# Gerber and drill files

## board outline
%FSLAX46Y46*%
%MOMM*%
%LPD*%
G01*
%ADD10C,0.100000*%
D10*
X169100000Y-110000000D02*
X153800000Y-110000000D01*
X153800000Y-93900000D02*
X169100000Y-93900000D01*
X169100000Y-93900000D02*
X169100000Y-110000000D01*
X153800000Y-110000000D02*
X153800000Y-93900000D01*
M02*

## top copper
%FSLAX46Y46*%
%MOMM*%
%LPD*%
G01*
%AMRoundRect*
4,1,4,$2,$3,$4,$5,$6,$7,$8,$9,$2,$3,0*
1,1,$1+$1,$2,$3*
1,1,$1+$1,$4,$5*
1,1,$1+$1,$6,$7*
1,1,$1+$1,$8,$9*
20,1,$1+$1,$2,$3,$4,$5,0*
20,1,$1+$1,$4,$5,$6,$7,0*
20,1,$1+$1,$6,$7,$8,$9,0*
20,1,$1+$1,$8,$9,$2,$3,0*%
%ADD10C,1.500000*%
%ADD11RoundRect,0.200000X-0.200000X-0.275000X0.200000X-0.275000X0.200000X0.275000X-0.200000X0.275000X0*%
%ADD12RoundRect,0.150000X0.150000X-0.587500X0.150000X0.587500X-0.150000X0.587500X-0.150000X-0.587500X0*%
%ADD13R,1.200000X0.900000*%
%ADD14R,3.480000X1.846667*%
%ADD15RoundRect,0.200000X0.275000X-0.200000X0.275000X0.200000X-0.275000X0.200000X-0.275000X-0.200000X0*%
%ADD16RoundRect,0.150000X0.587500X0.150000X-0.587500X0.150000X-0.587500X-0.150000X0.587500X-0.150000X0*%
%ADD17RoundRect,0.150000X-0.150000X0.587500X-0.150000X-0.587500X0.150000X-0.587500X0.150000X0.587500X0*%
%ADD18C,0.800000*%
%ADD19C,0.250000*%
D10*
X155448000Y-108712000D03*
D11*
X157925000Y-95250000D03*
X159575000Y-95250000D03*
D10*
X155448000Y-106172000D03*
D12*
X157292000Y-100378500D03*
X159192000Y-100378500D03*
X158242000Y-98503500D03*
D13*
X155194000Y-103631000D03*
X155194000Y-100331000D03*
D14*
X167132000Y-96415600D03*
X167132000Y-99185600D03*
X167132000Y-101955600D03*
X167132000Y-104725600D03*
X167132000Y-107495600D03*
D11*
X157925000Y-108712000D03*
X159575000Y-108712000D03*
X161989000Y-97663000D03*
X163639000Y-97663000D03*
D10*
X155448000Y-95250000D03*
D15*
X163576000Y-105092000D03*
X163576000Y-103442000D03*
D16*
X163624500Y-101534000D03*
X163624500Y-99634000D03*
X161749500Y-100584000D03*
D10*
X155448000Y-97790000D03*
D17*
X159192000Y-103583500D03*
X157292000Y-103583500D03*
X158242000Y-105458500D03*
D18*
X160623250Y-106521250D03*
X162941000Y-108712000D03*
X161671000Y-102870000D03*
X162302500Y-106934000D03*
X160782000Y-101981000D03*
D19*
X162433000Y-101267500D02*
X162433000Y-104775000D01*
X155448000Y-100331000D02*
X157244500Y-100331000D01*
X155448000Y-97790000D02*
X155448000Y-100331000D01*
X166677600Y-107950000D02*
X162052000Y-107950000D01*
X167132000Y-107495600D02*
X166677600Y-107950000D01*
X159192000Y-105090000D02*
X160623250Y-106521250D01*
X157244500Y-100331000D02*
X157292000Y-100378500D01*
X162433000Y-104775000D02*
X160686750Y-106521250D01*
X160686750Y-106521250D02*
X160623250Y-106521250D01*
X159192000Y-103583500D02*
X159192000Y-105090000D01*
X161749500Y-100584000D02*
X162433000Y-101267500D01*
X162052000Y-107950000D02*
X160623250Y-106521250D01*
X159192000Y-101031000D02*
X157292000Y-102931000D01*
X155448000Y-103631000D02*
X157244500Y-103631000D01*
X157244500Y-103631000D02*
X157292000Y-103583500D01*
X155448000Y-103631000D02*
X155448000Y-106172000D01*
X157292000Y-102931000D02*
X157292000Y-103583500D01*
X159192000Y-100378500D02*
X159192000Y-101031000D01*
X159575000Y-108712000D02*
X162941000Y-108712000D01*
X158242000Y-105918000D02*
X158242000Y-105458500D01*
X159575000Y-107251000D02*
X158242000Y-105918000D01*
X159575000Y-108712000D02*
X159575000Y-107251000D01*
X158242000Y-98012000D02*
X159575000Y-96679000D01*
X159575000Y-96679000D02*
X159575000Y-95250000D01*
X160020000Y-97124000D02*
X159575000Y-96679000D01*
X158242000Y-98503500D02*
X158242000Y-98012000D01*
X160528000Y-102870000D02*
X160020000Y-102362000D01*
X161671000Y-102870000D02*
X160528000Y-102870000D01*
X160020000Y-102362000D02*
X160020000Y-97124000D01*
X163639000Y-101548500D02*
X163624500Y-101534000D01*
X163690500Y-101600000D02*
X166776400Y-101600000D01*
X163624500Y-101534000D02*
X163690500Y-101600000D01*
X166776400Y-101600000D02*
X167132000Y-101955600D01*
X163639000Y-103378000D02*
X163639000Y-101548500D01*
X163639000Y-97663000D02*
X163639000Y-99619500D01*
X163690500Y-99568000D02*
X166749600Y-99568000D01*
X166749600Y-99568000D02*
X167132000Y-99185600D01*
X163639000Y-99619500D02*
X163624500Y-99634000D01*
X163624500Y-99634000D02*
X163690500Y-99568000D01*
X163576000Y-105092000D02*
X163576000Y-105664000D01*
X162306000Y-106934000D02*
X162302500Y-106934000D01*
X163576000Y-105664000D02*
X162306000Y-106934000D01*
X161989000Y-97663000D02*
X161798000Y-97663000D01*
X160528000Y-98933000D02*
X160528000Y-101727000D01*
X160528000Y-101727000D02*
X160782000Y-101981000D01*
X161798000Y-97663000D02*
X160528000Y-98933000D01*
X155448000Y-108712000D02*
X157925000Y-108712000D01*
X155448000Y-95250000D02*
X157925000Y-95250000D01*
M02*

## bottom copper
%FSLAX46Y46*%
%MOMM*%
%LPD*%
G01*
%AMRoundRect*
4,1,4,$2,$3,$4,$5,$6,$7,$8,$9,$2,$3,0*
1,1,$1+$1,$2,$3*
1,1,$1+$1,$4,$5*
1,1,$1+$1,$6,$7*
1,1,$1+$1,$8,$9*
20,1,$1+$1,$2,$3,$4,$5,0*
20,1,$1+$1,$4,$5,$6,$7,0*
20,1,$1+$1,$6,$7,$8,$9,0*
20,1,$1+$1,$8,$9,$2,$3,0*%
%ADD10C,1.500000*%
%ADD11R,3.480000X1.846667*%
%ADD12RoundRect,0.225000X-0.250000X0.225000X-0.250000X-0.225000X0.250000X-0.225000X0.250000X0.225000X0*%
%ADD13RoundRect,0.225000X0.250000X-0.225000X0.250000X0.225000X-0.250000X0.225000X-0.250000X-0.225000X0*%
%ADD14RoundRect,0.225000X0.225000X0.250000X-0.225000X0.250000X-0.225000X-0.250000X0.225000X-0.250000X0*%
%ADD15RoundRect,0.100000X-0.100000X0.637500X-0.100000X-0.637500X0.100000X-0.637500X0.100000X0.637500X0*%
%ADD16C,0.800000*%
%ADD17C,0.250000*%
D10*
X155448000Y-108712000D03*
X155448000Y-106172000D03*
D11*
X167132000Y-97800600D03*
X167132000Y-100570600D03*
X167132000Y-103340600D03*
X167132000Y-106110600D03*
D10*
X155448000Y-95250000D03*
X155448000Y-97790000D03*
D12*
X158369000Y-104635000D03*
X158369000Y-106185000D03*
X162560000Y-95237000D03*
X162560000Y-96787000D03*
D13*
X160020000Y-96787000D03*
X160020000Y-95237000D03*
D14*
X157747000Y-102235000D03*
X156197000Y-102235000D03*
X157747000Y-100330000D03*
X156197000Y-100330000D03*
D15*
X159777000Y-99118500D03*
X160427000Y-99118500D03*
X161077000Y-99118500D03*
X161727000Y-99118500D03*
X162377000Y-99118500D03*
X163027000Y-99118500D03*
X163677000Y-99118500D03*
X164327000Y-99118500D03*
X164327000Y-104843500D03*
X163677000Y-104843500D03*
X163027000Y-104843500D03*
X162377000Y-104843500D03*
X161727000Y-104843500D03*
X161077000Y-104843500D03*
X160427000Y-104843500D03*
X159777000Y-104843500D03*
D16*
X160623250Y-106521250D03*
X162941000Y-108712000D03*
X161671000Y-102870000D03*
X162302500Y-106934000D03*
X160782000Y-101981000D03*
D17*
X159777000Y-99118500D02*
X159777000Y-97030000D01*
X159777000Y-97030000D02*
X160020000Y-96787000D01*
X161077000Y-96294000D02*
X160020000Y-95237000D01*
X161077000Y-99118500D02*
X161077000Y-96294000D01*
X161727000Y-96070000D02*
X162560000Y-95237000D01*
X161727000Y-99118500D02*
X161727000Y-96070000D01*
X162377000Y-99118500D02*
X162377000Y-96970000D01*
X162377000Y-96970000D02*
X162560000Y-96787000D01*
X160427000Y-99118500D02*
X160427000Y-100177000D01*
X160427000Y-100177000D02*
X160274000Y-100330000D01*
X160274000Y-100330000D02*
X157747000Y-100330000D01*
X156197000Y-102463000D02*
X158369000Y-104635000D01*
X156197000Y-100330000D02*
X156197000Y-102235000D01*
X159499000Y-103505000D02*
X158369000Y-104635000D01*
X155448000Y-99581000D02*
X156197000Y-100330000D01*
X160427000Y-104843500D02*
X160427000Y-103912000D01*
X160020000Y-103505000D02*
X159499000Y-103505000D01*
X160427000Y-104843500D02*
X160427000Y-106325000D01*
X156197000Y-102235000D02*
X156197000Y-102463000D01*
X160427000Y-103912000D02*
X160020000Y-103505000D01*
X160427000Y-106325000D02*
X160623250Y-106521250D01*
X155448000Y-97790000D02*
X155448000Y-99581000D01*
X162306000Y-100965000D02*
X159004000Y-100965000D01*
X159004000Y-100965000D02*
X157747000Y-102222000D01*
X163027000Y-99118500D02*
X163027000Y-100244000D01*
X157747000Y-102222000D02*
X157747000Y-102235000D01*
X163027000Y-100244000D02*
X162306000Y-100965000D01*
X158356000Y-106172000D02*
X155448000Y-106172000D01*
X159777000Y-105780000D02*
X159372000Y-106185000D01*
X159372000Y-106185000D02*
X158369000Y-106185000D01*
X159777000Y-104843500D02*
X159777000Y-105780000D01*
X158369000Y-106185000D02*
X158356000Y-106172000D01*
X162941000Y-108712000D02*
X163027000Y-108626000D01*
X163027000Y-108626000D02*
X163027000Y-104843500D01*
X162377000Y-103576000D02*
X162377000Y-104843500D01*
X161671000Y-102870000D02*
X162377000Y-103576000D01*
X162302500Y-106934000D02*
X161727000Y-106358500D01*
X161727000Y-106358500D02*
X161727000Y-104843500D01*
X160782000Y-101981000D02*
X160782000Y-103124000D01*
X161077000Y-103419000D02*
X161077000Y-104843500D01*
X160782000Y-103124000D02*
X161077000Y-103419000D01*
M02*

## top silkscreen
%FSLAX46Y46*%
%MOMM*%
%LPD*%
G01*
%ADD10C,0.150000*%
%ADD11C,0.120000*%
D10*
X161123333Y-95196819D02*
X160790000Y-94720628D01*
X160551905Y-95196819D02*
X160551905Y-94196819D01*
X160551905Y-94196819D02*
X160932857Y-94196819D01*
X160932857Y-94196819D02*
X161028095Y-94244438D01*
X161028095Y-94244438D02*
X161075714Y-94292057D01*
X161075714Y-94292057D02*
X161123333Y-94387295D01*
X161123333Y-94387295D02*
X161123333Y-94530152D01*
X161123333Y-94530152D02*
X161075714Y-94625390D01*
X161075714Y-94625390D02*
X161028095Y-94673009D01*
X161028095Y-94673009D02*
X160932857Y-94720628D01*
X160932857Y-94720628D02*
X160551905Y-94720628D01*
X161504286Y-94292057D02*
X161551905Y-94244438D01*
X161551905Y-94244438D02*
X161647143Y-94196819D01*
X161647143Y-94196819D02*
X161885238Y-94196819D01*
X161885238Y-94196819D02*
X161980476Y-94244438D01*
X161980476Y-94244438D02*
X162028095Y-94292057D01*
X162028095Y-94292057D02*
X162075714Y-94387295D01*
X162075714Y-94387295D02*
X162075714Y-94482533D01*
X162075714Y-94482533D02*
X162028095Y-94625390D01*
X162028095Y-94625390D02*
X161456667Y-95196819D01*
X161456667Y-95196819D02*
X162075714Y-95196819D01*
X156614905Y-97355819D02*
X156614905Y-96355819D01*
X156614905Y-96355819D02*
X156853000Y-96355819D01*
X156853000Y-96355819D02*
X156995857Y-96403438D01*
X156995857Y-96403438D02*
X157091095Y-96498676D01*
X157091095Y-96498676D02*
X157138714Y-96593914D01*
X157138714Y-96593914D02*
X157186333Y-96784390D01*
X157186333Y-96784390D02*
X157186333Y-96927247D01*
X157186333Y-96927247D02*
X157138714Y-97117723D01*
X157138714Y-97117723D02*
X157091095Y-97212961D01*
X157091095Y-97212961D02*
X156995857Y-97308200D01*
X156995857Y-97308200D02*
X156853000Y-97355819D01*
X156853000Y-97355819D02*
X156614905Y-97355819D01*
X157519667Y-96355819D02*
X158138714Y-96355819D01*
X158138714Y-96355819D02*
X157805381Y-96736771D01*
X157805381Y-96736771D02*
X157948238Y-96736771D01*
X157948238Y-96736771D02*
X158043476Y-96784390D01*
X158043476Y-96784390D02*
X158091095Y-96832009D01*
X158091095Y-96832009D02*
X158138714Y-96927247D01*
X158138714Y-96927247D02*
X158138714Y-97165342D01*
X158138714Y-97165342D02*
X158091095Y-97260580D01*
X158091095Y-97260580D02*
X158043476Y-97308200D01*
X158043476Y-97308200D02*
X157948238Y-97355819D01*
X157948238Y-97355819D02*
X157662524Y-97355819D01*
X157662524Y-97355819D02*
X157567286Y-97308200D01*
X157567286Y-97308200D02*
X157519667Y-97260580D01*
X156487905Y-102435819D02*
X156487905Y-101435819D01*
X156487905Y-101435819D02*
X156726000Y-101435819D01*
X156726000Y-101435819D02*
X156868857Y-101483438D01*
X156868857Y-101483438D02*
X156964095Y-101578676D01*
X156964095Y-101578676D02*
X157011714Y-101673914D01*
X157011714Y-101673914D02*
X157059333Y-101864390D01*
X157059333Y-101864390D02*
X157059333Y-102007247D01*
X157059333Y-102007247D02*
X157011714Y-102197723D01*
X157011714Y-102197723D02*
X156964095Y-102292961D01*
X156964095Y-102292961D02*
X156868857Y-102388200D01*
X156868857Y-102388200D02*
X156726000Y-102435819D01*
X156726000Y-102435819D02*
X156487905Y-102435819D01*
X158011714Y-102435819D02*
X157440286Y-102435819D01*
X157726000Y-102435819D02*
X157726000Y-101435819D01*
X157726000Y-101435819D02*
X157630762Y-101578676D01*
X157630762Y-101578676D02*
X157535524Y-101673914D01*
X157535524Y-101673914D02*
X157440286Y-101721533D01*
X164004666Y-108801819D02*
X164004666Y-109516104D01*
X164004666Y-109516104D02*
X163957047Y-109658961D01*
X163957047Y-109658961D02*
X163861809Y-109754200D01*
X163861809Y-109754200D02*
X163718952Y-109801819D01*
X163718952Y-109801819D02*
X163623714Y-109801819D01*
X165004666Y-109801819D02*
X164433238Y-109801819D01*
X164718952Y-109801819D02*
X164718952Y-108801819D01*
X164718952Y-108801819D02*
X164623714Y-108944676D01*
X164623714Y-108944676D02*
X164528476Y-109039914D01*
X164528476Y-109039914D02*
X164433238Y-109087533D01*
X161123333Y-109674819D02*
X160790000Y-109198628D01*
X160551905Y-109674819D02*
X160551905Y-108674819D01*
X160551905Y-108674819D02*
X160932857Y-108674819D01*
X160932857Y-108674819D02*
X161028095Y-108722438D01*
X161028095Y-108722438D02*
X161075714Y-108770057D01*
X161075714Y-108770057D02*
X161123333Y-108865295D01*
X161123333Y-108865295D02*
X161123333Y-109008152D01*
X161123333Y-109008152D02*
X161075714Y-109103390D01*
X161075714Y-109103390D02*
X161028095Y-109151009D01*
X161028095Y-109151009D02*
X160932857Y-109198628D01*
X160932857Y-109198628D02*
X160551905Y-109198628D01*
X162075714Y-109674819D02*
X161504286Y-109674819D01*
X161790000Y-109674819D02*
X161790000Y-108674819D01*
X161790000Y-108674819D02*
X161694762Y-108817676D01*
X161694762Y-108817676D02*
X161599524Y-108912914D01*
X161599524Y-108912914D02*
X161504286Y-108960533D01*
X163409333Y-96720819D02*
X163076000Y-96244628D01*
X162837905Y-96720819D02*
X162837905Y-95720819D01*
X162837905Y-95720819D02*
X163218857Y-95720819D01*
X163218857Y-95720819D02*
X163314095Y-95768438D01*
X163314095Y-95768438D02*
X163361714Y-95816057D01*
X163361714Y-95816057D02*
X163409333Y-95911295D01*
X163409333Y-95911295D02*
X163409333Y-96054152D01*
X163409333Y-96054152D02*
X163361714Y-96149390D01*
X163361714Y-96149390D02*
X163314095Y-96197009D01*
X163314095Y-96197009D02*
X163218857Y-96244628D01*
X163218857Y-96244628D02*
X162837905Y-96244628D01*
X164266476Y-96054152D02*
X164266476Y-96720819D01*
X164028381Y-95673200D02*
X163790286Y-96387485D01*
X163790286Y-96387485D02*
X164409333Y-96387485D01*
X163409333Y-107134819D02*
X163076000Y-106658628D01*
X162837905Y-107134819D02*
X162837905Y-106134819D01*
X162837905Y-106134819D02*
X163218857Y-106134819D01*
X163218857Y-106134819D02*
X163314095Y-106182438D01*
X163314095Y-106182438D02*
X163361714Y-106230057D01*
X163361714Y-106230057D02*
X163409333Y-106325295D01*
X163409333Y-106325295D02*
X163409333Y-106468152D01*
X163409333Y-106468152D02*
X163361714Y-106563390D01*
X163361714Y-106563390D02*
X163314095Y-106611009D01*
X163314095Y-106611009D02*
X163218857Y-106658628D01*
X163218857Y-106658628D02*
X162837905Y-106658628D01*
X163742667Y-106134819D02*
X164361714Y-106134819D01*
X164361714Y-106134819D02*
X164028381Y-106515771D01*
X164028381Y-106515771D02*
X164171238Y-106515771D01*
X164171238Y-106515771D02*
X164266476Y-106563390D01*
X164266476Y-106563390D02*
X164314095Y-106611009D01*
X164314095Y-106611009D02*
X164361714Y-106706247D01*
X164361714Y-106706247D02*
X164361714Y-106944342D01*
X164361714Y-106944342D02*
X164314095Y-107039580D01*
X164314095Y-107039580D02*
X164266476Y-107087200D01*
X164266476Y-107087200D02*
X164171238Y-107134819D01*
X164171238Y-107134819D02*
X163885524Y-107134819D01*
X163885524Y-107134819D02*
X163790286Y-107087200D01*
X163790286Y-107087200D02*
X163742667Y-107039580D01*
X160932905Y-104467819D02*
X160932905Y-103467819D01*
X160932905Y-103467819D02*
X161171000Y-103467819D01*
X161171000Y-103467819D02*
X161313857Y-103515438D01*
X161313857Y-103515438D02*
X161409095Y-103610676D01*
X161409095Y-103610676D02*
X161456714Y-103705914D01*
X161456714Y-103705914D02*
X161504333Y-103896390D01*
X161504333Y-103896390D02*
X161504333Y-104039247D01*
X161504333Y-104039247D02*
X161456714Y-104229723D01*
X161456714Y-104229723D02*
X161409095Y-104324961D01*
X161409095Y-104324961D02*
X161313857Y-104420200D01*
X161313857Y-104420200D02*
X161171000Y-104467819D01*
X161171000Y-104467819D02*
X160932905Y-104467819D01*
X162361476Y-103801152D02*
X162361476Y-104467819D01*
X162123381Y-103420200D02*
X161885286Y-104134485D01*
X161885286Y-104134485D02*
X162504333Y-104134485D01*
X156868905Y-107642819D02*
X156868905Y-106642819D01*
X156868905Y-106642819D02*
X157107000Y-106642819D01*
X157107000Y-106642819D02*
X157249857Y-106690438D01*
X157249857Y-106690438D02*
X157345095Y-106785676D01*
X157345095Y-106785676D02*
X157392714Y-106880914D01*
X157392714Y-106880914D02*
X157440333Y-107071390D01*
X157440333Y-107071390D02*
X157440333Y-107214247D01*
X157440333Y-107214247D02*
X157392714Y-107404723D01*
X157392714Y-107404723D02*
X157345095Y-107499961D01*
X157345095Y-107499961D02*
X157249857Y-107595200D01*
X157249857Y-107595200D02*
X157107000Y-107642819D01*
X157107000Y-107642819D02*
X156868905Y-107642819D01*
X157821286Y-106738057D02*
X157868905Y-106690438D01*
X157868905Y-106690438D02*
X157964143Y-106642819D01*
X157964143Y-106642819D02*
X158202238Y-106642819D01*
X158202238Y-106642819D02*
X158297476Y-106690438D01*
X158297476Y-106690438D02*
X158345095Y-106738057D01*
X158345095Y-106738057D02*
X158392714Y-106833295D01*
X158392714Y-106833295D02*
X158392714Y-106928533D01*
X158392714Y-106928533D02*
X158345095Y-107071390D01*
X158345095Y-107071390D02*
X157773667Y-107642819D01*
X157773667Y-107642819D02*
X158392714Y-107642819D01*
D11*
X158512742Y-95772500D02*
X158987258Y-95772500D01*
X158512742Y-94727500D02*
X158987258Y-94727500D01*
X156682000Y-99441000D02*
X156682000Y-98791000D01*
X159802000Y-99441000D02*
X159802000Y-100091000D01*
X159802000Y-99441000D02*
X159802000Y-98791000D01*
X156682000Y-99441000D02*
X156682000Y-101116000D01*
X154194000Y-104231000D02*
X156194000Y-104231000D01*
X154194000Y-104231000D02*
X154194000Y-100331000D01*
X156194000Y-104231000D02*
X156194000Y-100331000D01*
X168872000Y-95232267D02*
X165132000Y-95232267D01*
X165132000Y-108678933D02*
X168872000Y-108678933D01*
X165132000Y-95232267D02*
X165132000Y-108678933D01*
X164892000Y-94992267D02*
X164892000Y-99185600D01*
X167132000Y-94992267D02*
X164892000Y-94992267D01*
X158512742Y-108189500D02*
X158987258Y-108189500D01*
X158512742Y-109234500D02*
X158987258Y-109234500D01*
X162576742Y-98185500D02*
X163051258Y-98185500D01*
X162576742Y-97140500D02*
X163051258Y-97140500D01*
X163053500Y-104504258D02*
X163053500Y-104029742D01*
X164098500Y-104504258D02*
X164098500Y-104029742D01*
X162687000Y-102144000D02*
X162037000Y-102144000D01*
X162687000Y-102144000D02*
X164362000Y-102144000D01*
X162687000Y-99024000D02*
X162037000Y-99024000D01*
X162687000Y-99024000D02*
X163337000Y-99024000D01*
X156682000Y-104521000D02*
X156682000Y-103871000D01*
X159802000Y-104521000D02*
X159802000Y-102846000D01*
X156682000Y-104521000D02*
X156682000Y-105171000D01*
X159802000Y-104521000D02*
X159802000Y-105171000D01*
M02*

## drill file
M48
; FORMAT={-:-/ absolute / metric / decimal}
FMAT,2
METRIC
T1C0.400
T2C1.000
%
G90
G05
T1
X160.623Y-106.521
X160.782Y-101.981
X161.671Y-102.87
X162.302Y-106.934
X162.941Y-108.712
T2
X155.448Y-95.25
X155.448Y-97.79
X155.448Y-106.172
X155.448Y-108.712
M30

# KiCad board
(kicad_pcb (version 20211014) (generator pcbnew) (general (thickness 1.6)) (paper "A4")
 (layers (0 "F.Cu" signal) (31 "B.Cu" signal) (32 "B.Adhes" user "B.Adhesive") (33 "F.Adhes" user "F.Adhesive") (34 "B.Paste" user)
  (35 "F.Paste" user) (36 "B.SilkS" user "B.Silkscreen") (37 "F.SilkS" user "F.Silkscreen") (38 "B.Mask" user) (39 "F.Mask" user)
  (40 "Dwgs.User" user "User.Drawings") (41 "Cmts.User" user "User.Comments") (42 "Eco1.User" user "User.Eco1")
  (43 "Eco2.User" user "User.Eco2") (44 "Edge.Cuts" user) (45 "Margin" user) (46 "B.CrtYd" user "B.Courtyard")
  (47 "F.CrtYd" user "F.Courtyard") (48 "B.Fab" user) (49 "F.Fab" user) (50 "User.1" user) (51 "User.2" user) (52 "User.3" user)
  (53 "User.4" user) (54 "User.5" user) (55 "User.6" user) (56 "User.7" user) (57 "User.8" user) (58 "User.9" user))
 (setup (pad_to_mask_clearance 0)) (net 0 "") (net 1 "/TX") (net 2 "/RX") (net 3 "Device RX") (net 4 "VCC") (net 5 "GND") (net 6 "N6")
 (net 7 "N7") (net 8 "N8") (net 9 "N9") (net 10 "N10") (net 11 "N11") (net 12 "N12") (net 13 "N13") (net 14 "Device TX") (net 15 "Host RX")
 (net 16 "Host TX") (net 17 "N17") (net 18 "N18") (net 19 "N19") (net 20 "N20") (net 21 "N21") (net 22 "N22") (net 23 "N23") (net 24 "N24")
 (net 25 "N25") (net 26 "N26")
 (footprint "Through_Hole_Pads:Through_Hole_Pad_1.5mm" (layer "F.Cu") (at 155.448 108.712)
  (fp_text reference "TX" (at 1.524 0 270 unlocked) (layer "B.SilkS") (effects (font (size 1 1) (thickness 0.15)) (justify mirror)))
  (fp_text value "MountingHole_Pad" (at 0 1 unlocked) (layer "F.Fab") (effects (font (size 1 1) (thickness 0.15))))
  (pad "1" thru_hole circle (at 0 0) (size 1.5 1.5) (drill 1) (layers *.Cu *.Mask) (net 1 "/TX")))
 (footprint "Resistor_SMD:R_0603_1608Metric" (layer "F.Cu") (at 158.75 95.25)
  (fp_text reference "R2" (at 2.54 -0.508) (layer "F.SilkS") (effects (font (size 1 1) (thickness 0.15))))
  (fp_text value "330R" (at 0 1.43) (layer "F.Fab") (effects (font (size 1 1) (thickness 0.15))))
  (fp_line (start -0.237258 0.5225) (end 0.237258 0.5225) (layer "F.SilkS") (width 0.12))
  (fp_line (start -0.237258 -0.5225) (end 0.237258 -0.5225) (layer "F.SilkS") (width 0.12))
  (pad "1" smd roundrect locked (at -0.825 0) (size 0.8 0.95) (layers "F.Cu" "F.Paste" "F.Mask") (roundrect_rratio 0.25) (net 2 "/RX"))
  (pad "2" smd roundrect locked (at 0.825 0) (size 0.8 0.95) (layers "F.Cu" "F.Paste" "F.Mask") (roundrect_rratio 0.25) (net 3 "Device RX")))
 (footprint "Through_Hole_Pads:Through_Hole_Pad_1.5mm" (layer "F.Cu") (at 155.448 106.172)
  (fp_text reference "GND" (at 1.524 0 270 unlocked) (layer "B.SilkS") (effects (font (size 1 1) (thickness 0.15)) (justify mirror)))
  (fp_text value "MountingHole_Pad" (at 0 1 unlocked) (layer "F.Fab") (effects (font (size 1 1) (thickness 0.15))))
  (pad "1" thru_hole circle (at 0 0) (size 1.5 1.5) (drill 1) (layers *.Cu *.Mask) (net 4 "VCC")))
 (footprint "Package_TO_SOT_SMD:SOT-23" (layer "F.Cu") (at 158.242 99.441 90)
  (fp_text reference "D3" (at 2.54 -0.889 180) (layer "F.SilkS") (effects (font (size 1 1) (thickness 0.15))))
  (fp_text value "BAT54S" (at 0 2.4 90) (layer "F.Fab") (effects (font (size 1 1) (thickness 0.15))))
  (fp_line (start 0 -1.56) (end 0.65 -1.56) (layer "F.SilkS") (width 0.12))
  (fp_line (start 0 1.56) (end -0.65 1.56) (layer "F.SilkS") (width 0.12))
  (fp_line (start 0 1.56) (end 0.65 1.56) (layer "F.SilkS") (width 0.12))
  (fp_line (start 0 -1.56) (end -1.675 -1.56) (layer "F.SilkS") (width 0.12))
  (pad "1" smd roundrect locked (at -0.9375 -0.95 90) (size 1.475 0.6) (layers "F.Cu" "F.Paste" "F.Mask") (roundrect_rratio 0.25)
   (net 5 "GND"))
  (pad "2" smd roundrect locked (at -0.9375 0.95 90) (size 1.475 0.6) (layers "F.Cu" "F.Paste" "F.Mask") (roundrect_rratio 0.25)
   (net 4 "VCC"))
  (pad "3" smd roundrect locked (at 0.9375 0 90) (size 1.475 0.6) (layers "F.Cu" "F.Paste" "F.Mask") (roundrect_rratio 0.25)
   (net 3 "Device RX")))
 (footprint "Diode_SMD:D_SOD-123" (layer "F.Cu") (at 155.194 101.981 90)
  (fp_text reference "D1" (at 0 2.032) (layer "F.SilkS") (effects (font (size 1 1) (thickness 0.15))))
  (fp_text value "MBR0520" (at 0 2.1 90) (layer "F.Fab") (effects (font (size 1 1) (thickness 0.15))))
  (fp_line (start -2.25 -1) (end -2.25 1) (layer "F.SilkS") (width 0.12))
  (fp_line (start -2.25 -1) (end 1.65 -1) (layer "F.SilkS") (width 0.12))
  (fp_line (start -2.25 1) (end 1.65 1) (layer "F.SilkS") (width 0.12))
  (pad "1" smd rect locked (at -1.65 0 90) (size 0.9 1.2) (layers "F.Cu" "F.Paste" "F.Mask") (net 4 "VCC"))
  (pad "2" smd rect locked (at 1.65 0 90) (size 0.9 1.2) (layers "F.Cu" "F.Paste" "F.Mask") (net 5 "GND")))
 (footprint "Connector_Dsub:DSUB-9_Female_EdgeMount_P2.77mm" (layer "F.Cu") (at 167.132 101.9556 90)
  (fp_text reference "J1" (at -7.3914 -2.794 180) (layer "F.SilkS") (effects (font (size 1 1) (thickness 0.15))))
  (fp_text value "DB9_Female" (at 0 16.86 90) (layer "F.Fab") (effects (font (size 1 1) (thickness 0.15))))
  (fp_line (start 6.723333 1.74) (end 6.723333 -2) (layer "F.SilkS") (width 0.12))
  (fp_line (start -6.723333 -2) (end -6.723333 1.74) (layer "F.SilkS") (width 0.12))
  (fp_line (start 6.723333 -2) (end -6.723333 -2) (layer "F.SilkS") (width 0.12))
  (fp_line (start 6.963333 -2.24) (end 2.77 -2.24) (layer "F.SilkS") (width 0.12))
  (fp_line (start 6.963333 0) (end 6.963333 -2.24) (layer "F.SilkS") (width 0.12))
  (pad "1" smd rect locked (at 5.54 0 90) (size 1.846667 3.48) (layers "F.Cu" "F.Paste" "F.Mask") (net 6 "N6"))
  (pad "2" smd rect locked (at 2.77 0 90) (size 1.846667 3.48) (layers "F.Cu" "F.Paste" "F.Mask") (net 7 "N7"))
  (pad "3" smd rect locked (at 0 0 90) (size 1.846667 3.48) (layers "F.Cu" "F.Paste" "F.Mask") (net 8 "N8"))
  (pad "4" smd rect locked (at -2.77 0 90) (size 1.846667 3.48) (layers "F.Cu" "F.Paste" "F.Mask") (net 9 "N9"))
  (pad "5" smd rect locked (at -5.54 0 90) (size 1.846667 3.48) (layers "F.Cu" "F.Paste" "F.Mask") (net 5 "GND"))
  (pad "6" smd rect locked (at 4.155 0 90) (size 1.846667 3.48) (layers "B.Cu" "B.Paste" "B.Mask") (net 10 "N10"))
  (pad "7" smd rect locked (at 1.385 0 90) (size 1.846667 3.48) (layers "B.Cu" "B.Paste" "B.Mask") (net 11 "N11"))
  (pad "8" smd rect locked (at -1.385 0 90) (size 1.846667 3.48) (layers "B.Cu" "B.Paste" "B.Mask") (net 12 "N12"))
  (pad "9" smd rect locked (at -4.155 0 90) (size 1.846667 3.48) (layers "B.Cu" "B.Paste" "B.Mask") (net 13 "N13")))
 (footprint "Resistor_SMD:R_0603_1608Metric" (layer "F.Cu") (at 158.75 108.712)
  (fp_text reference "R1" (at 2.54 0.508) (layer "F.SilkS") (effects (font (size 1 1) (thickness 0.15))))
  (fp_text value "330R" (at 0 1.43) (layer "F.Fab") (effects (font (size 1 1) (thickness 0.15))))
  (fp_line (start -0.237258 -0.5225) (end 0.237258 -0.5225) (layer "F.SilkS") (width 0.12))
  (fp_line (start -0.237258 0.5225) (end 0.237258 0.5225) (layer "F.SilkS") (width 0.12))
  (pad "1" smd roundrect locked (at -0.825 0) (size 0.8 0.95) (layers "F.Cu" "F.Paste" "F.Mask") (roundrect_rratio 0.25) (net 1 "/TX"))
  (pad "2" smd roundrect locked (at 0.825 0) (size 0.8 0.95) (layers "F.Cu" "F.Paste" "F.Mask") (roundrect_rratio 0.25) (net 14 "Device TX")))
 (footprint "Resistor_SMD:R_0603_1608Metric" (layer "F.Cu") (at 162.814 97.663)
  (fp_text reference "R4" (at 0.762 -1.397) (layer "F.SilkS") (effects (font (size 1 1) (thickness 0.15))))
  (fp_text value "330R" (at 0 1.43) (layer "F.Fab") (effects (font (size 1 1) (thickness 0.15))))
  (fp_line (start -0.237258 0.5225) (end 0.237258 0.5225) (layer "F.SilkS") (width 0.12))
  (fp_line (start -0.237258 -0.5225) (end 0.237258 -0.5225) (layer "F.SilkS") (width 0.12))
  (pad "1" smd roundrect locked (at -0.825 0) (size 0.8 0.95) (layers "F.Cu" "F.Paste" "F.Mask") (roundrect_rratio 0.25) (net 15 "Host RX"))
  (pad "2" smd roundrect locked (at 0.825 0) (size 0.8 0.95) (layers "F.Cu" "F.Paste" "F.Mask") (roundrect_rratio 0.25) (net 7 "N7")))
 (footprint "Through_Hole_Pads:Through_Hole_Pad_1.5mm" (layer "F.Cu") (at 155.448 95.25)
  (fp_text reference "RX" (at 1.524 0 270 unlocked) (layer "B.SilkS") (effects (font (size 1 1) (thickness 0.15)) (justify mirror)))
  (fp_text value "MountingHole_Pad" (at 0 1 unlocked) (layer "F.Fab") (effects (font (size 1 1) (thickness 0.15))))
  (pad "1" thru_hole circle (at 0 0) (size 1.5 1.5) (drill 1) (layers *.Cu *.Mask) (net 2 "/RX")))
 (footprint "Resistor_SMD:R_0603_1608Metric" (layer "F.Cu") (at 163.576 104.267 90)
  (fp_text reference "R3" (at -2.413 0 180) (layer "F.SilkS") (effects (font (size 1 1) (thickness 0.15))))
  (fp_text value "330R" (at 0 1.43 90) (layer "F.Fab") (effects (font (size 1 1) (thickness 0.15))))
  (fp_line (start -0.237258 -0.5225) (end 0.237258 -0.5225) (layer "F.SilkS") (width 0.12))
  (fp_line (start -0.237258 0.5225) (end 0.237258 0.5225) (layer "F.SilkS") (width 0.12))
  (pad "1" smd roundrect locked (at -0.825 0 90) (size 0.8 0.95) (layers "F.Cu" "F.Paste" "F.Mask") (roundrect_rratio 0.25)
   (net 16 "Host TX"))
  (pad "2" smd roundrect locked (at 0.825 0 90) (size 0.8 0.95) (layers "F.Cu" "F.Paste" "F.Mask") (roundrect_rratio 0.25) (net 8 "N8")))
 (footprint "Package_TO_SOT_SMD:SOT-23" (layer "F.Cu") (at 162.687 100.584 180)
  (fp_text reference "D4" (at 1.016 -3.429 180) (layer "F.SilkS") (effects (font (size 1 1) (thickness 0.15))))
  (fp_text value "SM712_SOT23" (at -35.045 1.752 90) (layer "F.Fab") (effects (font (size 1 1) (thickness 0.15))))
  (fp_line (start 0 -1.56) (end 0.65 -1.56) (layer "F.SilkS") (width 0.12))
  (fp_line (start 0 -1.56) (end -1.675 -1.56) (layer "F.SilkS") (width 0.12))
  (fp_line (start 0 1.56) (end 0.65 1.56) (layer "F.SilkS") (width 0.12))
  (fp_line (start 0 1.56) (end -0.65 1.56) (layer "F.SilkS") (width 0.12))
  (pad "1" smd roundrect locked (at -0.9375 -0.95 180) (size 1.475 0.6) (layers "F.Cu" "F.Paste" "F.Mask") (roundrect_rratio 0.25)
   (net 8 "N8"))
  (pad "2" smd roundrect locked (at -0.9375 0.95 180) (size 1.475 0.6) (layers "F.Cu" "F.Paste" "F.Mask") (roundrect_rratio 0.25)
   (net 7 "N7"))
  (pad "3" smd roundrect locked (at 0.9375 0 180) (size 1.475 0.6) (layers "F.Cu" "F.Paste" "F.Mask") (roundrect_rratio 0.25) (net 5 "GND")))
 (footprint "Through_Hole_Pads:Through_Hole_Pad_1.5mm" (layer "F.Cu") (at 155.448 97.79 180)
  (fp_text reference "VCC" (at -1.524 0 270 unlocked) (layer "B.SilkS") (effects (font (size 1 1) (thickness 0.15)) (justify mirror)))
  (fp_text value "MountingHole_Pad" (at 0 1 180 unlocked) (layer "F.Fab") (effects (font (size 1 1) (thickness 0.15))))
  (pad "1" thru_hole circle (at 0 0 180) (size 1.5 1.5) (drill 1) (layers *.Cu *.Mask) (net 5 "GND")))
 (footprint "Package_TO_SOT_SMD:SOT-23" (layer "F.Cu") (at 158.242 104.521 -90)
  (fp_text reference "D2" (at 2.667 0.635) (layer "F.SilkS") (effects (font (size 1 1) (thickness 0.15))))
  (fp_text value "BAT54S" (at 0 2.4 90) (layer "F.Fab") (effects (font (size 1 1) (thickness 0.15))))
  (fp_line (start 0 1.56) (end -0.65 1.56) (layer "F.SilkS") (width 0.12))
  (fp_line (start 0 -1.56) (end -1.675 -1.56) (layer "F.SilkS") (width 0.12))
  (fp_line (start 0 1.56) (end 0.65 1.56) (layer "F.SilkS") (width 0.12))
  (fp_line (start 0 -1.56) (end 0.65 -1.56) (layer "F.SilkS") (width 0.12))
  (pad "1" smd roundrect locked (at -0.9375 -0.95 270) (size 1.475 0.6) (layers "F.Cu" "F.Paste" "F.Mask") (roundrect_rratio 0.25)
   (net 5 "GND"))
  (pad "2" smd roundrect locked (at -0.9375 0.95 270) (size 1.475 0.6) (layers "F.Cu" "F.Paste" "F.Mask") (roundrect_rratio 0.25)
   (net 4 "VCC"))
  (pad "3" smd roundrect locked (at 0.9375 0 270) (size 1.475 0.6) (layers "F.Cu" "F.Paste" "F.Mask") (roundrect_rratio 0.25)
   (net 14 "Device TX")))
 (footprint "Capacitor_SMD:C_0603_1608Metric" (layer "B.Cu") (at 158.369 105.41 -90)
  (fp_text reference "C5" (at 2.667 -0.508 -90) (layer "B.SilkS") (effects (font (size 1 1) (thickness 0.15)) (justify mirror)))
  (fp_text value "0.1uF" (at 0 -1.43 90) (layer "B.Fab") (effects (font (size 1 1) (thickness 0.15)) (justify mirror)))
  (pad "1" smd roundrect locked (at -0.775 0 270) (size 0.9 0.95) (layers "B.Cu" "B.Paste" "B.Mask") (roundrect_rratio 0.25) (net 5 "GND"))
  (pad "2" smd roundrect locked (at 0.775 0 270) (size 0.9 0.95) (layers "B.Cu" "B.Paste" "B.Mask") (roundrect_rratio 0.25) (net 4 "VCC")))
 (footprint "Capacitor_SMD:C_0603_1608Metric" (layer "B.Cu") (at 162.56 96.012 -90)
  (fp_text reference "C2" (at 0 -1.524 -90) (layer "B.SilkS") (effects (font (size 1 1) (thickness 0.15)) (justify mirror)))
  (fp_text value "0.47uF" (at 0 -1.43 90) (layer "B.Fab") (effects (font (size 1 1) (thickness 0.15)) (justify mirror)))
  (pad "1" smd roundrect locked (at -0.775 0 270) (size 0.9 0.95) (layers "B.Cu" "B.Paste" "B.Mask") (roundrect_rratio 0.25) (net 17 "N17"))
  (pad "2" smd roundrect locked (at 0.775 0 270) (size 0.9 0.95) (layers "B.Cu" "B.Paste" "B.Mask") (roundrect_rratio 0.25) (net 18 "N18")))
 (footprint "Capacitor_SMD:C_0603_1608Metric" (layer "B.Cu") (at 160.02 96.012 90)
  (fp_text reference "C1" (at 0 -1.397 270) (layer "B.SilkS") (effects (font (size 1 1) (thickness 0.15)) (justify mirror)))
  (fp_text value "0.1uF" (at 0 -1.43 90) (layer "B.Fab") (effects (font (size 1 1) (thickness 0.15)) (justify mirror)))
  (pad "1" smd roundrect locked (at -0.775 0 90) (size 0.9 0.95) (layers "B.Cu" "B.Paste" "B.Mask") (roundrect_rratio 0.25) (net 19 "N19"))
  (pad "2" smd roundrect locked (at 0.775 0 90) (size 0.9 0.95) (layers "B.Cu" "B.Paste" "B.Mask") (roundrect_rratio 0.25) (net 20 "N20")))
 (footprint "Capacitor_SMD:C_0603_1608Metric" (layer "B.Cu") (at 156.972 102.235 180)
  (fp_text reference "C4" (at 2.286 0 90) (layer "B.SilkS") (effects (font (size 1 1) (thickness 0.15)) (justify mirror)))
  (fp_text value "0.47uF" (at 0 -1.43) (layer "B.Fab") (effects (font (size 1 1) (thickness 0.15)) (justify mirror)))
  (pad "1" smd roundrect locked (at -0.775 0 180) (size 0.9 0.95) (layers "B.Cu" "B.Paste" "B.Mask") (roundrect_rratio 0.25) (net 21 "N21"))
  (pad "2" smd roundrect locked (at 0.775 0 180) (size 0.9 0.95) (layers "B.Cu" "B.Paste" "B.Mask") (roundrect_rratio 0.25) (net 5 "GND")))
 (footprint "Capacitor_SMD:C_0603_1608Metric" (layer "B.Cu") (at 156.972 100.33 180)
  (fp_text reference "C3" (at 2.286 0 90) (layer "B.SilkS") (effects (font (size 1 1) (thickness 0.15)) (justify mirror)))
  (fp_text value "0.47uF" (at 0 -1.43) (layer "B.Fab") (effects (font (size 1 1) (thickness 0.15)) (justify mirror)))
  (pad "1" smd roundrect locked (at -0.775 0 180) (size 0.9 0.95) (layers "B.Cu" "B.Paste" "B.Mask") (roundrect_rratio 0.25) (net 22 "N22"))
  (pad "2" smd roundrect locked (at 0.775 0 180) (size 0.9 0.95) (layers "B.Cu" "B.Paste" "B.Mask") (roundrect_rratio 0.25) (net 5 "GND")))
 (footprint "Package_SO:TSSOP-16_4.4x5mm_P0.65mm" (layer "B.Cu") (at 162.052 101.981 -90)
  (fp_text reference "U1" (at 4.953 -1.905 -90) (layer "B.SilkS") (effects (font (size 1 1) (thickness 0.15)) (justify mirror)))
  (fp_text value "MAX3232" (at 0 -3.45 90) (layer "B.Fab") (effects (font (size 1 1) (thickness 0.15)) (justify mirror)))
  (pad "1" smd roundrect locked (at -2.8625 2.275 270) (size 1.475 0.4) (layers "B.Cu" "B.Paste" "B.Mask") (roundrect_rratio 0.25)
   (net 19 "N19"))
  (pad "2" smd roundrect locked (at -2.8625 1.625 270) (size 1.475 0.4) (layers "B.Cu" "B.Paste" "B.Mask") (roundrect_rratio 0.25)
   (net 22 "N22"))
  (pad "3" smd roundrect locked (at -2.8625 0.975 270) (size 1.475 0.4) (layers "B.Cu" "B.Paste" "B.Mask") (roundrect_rratio 0.25)
   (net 20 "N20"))
  (pad "4" smd roundrect locked (at -2.8625 0.325 270) (size 1.475 0.4) (layers "B.Cu" "B.Paste" "B.Mask") (roundrect_rratio 0.25)
   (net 17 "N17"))
  (pad "5" smd roundrect locked (at -2.8625 -0.325 270) (size 1.475 0.4) (layers "B.Cu" "B.Paste" "B.Mask") (roundrect_rratio 0.25)
   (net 18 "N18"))
  (pad "6" smd roundrect locked (at -2.8625 -0.975 270) (size 1.475 0.4) (layers "B.Cu" "B.Paste" "B.Mask") (roundrect_rratio 0.25)
   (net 21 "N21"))
  (pad "7" smd roundrect locked (at -2.8625 -1.625 270) (size 1.475 0.4) (layers "B.Cu" "B.Paste" "B.Mask") (roundrect_rratio 0.25)
   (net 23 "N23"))
  (pad "8" smd roundrect locked (at -2.8625 -2.275 270) (size 1.475 0.4) (layers "B.Cu" "B.Paste" "B.Mask") (roundrect_rratio 0.25)
   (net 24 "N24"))
  (pad "9" smd roundrect locked (at 2.8625 -2.275 270) (size 1.475 0.4) (layers "B.Cu" "B.Paste" "B.Mask") (roundrect_rratio 0.25)
   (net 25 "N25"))
  (pad "10" smd roundrect locked (at 2.8625 -1.625 270) (size 1.475 0.4) (layers "B.Cu" "B.Paste" "B.Mask") (roundrect_rratio 0.25)
   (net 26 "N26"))
  (pad "11" smd roundrect locked (at 2.8625 -0.975 270) (size 1.475 0.4) (layers "B.Cu" "B.Paste" "B.Mask") (roundrect_rratio 0.25)
   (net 14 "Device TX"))
  (pad "12" smd roundrect locked (at 2.8625 -0.325 270) (size 1.475 0.4) (layers "B.Cu" "B.Paste" "B.Mask") (roundrect_rratio 0.25)
   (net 3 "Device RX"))
  (pad "13" smd roundrect locked (at 2.8625 0.325 270) (size 1.475 0.4) (layers "B.Cu" "B.Paste" "B.Mask") (roundrect_rratio 0.25)
   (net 16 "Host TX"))
  (pad "14" smd roundrect locked (at 2.8625 0.975 270) (size 1.475 0.4) (layers "B.Cu" "B.Paste" "B.Mask") (roundrect_rratio 0.25)
   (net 15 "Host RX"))
  (pad "15" smd roundrect locked (at 2.8625 1.625 270) (size 1.475 0.4) (layers "B.Cu" "B.Paste" "B.Mask") (roundrect_rratio 0.25)
   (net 5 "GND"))
  (pad "16" smd roundrect locked (at 2.8625 2.275 270) (size 1.475 0.4) (layers "B.Cu" "B.Paste" "B.Mask") (roundrect_rratio 0.25)
   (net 4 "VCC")))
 (gr_line (start 169.1 110) (end 153.8 110) (layer "Edge.Cuts") (width 0.1))
 (gr_line (start 153.8 93.9) (end 169.1 93.9) (layer "Edge.Cuts") (width 0.1))
 (gr_line (start 169.1 93.9) (end 169.1 110) (layer "Edge.Cuts") (width 0.1))
 (gr_line (start 153.8 110) (end 153.8 93.9) (layer "Edge.Cuts") (width 0.1))
 (segment (start 159.777 99.1185) (end 159.777 97.03) (width 0.25) (layer "B.Cu") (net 19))
 (segment (start 159.777 97.03) (end 160.02 96.787) (width 0.25) (layer "B.Cu") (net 19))
 (segment (start 161.077 96.294) (end 160.02 95.237) (width 0.25) (layer "B.Cu") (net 20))
 (segment (start 161.077 99.1185) (end 161.077 96.294) (width 0.25) (layer "B.Cu") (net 20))
 (segment (start 161.727 96.07) (end 162.56 95.237) (width 0.25) (layer "B.Cu") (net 17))
 (segment (start 161.727 99.1185) (end 161.727 96.07) (width 0.25) (layer "B.Cu") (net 17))
 (segment (start 162.377 99.1185) (end 162.377 96.97) (width 0.25) (layer "B.Cu") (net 18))
 (segment (start 162.377 96.97) (end 162.56 96.787) (width 0.25) (layer "B.Cu") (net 18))
 (segment (start 160.427 99.1185) (end 160.427 100.177) (width 0.25) (layer "B.Cu") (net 22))
 (segment (start 160.427 100.177) (end 160.274 100.33) (width 0.25) (layer "B.Cu") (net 22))
 (segment (start 160.274 100.33) (end 157.747 100.33) (width 0.25) (layer "B.Cu") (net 22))
 (segment (start 162.433 101.2675) (end 162.433 104.775) (width 0.25) (layer "F.Cu") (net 5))
 (segment (start 155.448 100.331) (end 157.2445 100.331) (width 0.25) (layer "F.Cu") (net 5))
 (segment (start 155.448 97.79) (end 155.448 100.331) (width 0.25) (layer "F.Cu") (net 5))
 (segment (start 166.6776 107.95) (end 162.052 107.95) (width 0.25) (layer "F.Cu") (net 5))
 (segment (start 167.132 107.4956) (end 166.6776 107.95) (width 0.25) (layer "F.Cu") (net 5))
 (segment (start 159.192 105.09) (end 160.62325 106.52125) (width 0.25) (layer "F.Cu") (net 5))
 (segment (start 157.2445 100.331) (end 157.292 100.3785) (width 0.25) (layer "F.Cu") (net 5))
 (segment (start 162.433 104.775) (end 160.68675 106.52125) (width 0.25) (layer "F.Cu") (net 5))
 (segment (start 160.68675 106.52125) (end 160.62325 106.52125) (width 0.25) (layer "F.Cu") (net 5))
 (segment (start 159.192 103.5835) (end 159.192 105.09) (width 0.25) (layer "F.Cu") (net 5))
 (segment (start 161.7495 100.584) (end 162.433 101.2675) (width 0.25) (layer "F.Cu") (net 5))
 (segment (start 162.052 107.95) (end 160.62325 106.52125) (width 0.25) (layer "F.Cu") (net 5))
 (via (at 160.62325 106.52125) (size 0.8) (drill 0.4) (layers "F.Cu" "B.Cu") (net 5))
 (segment (start 156.197 102.463) (end 158.369 104.635) (width 0.25) (layer "B.Cu") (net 5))
 (segment (start 156.197 100.33) (end 156.197 102.235) (width 0.25) (layer "B.Cu") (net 5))
 (segment (start 159.499 103.505) (end 158.369 104.635) (width 0.25) (layer "B.Cu") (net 5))
 (segment (start 155.448 99.581) (end 156.197 100.33) (width 0.25) (layer "B.Cu") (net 5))
 (segment (start 160.427 104.8435) (end 160.427 103.912) (width 0.25) (layer "B.Cu") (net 5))
 (segment (start 160.02 103.505) (end 159.499 103.505) (width 0.25) (layer "B.Cu") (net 5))
 (segment (start 160.427 104.8435) (end 160.427 106.325) (width 0.25) (layer "B.Cu") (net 5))
 (segment (start 156.197 102.235) (end 156.197 102.463) (width 0.25) (layer "B.Cu") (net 5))
 (segment (start 160.427 103.912) (end 160.02 103.505) (width 0.25) (layer "B.Cu") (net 5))
 (segment (start 160.427 106.325) (end 160.62325 106.52125) (width 0.25) (layer "B.Cu") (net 5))
 (segment (start 155.448 97.79) (end 155.448 99.581) (width 0.25) (layer "B.Cu") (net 5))
 (segment (start 162.306 100.965) (end 159.004 100.965) (width 0.25) (layer "B.Cu") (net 21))
 (segment (start 159.004 100.965) (end 157.747 102.222) (width 0.25) (layer "B.Cu") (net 21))
 (segment (start 163.027 99.1185) (end 163.027 100.244) (width 0.25) (layer "B.Cu") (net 21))
 (segment (start 157.747 102.222) (end 157.747 102.235) (width 0.25) (layer "B.Cu") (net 21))
 (segment (start 163.027 100.244) (end 162.306 100.965) (width 0.25) (layer "B.Cu") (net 21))
 (segment (start 159.192 101.031) (end 157.292 102.931) (width 0.25) (layer "F.Cu") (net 4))
 (segment (start 155.448 103.631) (end 157.2445 103.631) (width 0.25) (layer "F.Cu") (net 4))
 (segment (start 157.2445 103.631) (end 157.292 103.5835) (width 0.25) (layer "F.Cu") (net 4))
 (segment (start 155.448 103.631) (end 155.448 106.172) (width 0.25) (layer "F.Cu") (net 4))
 (segment (start 157.292 102.931) (end 157.292 103.5835) (width 0.25) (layer "F.Cu") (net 4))
 (segment (start 159.192 100.3785) (end 159.192 101.031) (width 0.25) (layer "F.Cu") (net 4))
 (segment (start 158.356 106.172) (end 155.448 106.172) (width 0.25) (layer "B.Cu") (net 4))
 (segment (start 159.777 105.78) (end 159.372 106.185) (width 0.25) (layer "B.Cu") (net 4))
 (segment (start 159.372 106.185) (end 158.369 106.185) (width 0.25) (layer "B.Cu") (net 4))
 (segment (start 159.777 104.8435) (end 159.777 105.78) (width 0.25) (layer "B.Cu") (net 4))
 (segment (start 158.369 106.185) (end 158.356 106.172) (width 0.25) (layer "B.Cu") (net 4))
 (segment (start 159.575 108.712) (end 162.941 108.712) (width 0.25) (layer "F.Cu") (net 14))
 (segment (start 158.242 105.918) (end 158.242 105.4585) (width 0.25) (layer "F.Cu") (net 14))
 (segment (start 159.575 107.251) (end 158.242 105.918) (width 0.25) (layer "F.Cu") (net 14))
 (segment (start 159.575 108.712) (end 159.575 107.251) (width 0.25) (layer "F.Cu") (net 14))
 (via (at 162.941 108.712) (size 0.8) (drill 0.4) (layers "F.Cu" "B.Cu") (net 14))
 (segment (start 162.941 108.712) (end 163.027 108.626) (width 0.25) (layer "B.Cu") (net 14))
 (segment (start 163.027 108.626) (end 163.027 104.8435) (width 0.25) (layer "B.Cu") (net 14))
 (segment (start 158.242 98.012) (end 159.575 96.679) (width 0.25) (layer "F.Cu") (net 3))
 (segment (start 159.575 96.679) (end 159.575 95.25) (width 0.25) (layer "F.Cu") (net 3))
 (segment (start 160.02 97.124) (end 159.575 96.679) (width 0.25) (layer "F.Cu") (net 3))
 (segment (start 158.242 98.5035) (end 158.242 98.012) (width 0.25) (layer "F.Cu") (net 3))
 (segment (start 160.528 102.87) (end 160.02 102.362) (width 0.25) (layer "F.Cu") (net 3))
 (segment (start 161.671 102.87) (end 160.528 102.87) (width 0.25) (layer "F.Cu") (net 3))
 (segment (start 160.02 102.362) (end 160.02 97.124) (width 0.25) (layer "F.Cu") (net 3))
 (via (at 161.671 102.87) (size 0.8) (drill 0.4) (layers "F.Cu" "B.Cu") (free) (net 3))
 (segment (start 162.377 103.576) (end 162.377 104.8435) (width 0.25) (layer "B.Cu") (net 3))
 (segment (start 161.671 102.87) (end 162.377 103.576) (width 0.25) (layer "B.Cu") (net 3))
 (segment (start 163.639 101.5485) (end 163.6245 101.534) (width 0.25) (layer "F.Cu") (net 8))
 (segment (start 163.6905 101.6) (end 166.7764 101.6) (width 0.25) (layer "F.Cu") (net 8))
 (segment (start 163.6245 101.534) (end 163.6905 101.6) (width 0.25) (layer "F.Cu") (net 8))
 (segment (start 166.7764 101.6) (end 167.132 101.9556) (width 0.25) (layer "F.Cu") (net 8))
 (segment (start 163.639 103.378) (end 163.639 101.5485) (width 0.25) (layer "F.Cu") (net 8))
 (segment (start 163.639 97.663) (end 163.639 99.6195) (width 0.25) (layer "F.Cu") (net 7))
 (segment (start 163.6905 99.568) (end 166.7496 99.568) (width 0.25) (layer "F.Cu") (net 7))
 (segment (start 166.7496 99.568) (end 167.132 99.1856) (width 0.25) (layer "F.Cu") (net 7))
 (segment (start 163.639 99.6195) (end 163.6245 99.634) (width 0.25) (layer "F.Cu") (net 7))
 (segment (start 163.6245 99.634) (end 163.6905 99.568) (width 0.25) (layer "F.Cu") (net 7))
 (segment (start 163.576 105.092) (end 163.576 105.664) (width 0.25) (layer "F.Cu") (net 16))
 (segment (start 162.306 106.934) (end 162.3025 106.934) (width 0.25) (layer "F.Cu") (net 16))
 (segment (start 163.576 105.664) (end 162.306 106.934) (width 0.25) (layer "F.Cu") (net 16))
 (via (at 162.3025 106.934) (size 0.8) (drill 0.4) (layers "F.Cu" "B.Cu") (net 16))
 (segment (start 162.3025 106.934) (end 161.727 106.3585) (width 0.25) (layer "B.Cu") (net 16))
 (segment (start 161.727 106.3585) (end 161.727 104.8435) (width 0.25) (layer "B.Cu") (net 16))
 (segment (start 161.989 97.663) (end 161.798 97.663) (width 0.25) (layer "F.Cu") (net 15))
 (segment (start 160.528 98.933) (end 160.528 101.727) (width 0.25) (layer "F.Cu") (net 15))
 (segment (start 160.528 101.727) (end 160.782 101.981) (width 0.25) (layer "F.Cu") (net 15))
 (segment (start 161.798 97.663) (end 160.528 98.933) (width 0.25) (layer "F.Cu") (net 15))
 (via (at 160.782 101.981) (size 0.8) (drill 0.4) (layers "F.Cu" "B.Cu") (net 15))
 (segment (start 160.782 101.981) (end 160.782 103.124) (width 0.25) (layer "B.Cu") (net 15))
 (segment (start 161.077 103.419) (end 161.077 104.8435) (width 0.25) (layer "B.Cu") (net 15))
 (segment (start 160.782 103.124) (end 161.077 103.419) (width 0.25) (layer "B.Cu") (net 15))
 (segment (start 155.448 108.712) (end 157.925 108.712) (width 0.25) (layer "F.Cu") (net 1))
 (segment (start 155.448 95.25) (end 157.925 95.25) (width 0.25) (layer "F.Cu") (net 2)))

